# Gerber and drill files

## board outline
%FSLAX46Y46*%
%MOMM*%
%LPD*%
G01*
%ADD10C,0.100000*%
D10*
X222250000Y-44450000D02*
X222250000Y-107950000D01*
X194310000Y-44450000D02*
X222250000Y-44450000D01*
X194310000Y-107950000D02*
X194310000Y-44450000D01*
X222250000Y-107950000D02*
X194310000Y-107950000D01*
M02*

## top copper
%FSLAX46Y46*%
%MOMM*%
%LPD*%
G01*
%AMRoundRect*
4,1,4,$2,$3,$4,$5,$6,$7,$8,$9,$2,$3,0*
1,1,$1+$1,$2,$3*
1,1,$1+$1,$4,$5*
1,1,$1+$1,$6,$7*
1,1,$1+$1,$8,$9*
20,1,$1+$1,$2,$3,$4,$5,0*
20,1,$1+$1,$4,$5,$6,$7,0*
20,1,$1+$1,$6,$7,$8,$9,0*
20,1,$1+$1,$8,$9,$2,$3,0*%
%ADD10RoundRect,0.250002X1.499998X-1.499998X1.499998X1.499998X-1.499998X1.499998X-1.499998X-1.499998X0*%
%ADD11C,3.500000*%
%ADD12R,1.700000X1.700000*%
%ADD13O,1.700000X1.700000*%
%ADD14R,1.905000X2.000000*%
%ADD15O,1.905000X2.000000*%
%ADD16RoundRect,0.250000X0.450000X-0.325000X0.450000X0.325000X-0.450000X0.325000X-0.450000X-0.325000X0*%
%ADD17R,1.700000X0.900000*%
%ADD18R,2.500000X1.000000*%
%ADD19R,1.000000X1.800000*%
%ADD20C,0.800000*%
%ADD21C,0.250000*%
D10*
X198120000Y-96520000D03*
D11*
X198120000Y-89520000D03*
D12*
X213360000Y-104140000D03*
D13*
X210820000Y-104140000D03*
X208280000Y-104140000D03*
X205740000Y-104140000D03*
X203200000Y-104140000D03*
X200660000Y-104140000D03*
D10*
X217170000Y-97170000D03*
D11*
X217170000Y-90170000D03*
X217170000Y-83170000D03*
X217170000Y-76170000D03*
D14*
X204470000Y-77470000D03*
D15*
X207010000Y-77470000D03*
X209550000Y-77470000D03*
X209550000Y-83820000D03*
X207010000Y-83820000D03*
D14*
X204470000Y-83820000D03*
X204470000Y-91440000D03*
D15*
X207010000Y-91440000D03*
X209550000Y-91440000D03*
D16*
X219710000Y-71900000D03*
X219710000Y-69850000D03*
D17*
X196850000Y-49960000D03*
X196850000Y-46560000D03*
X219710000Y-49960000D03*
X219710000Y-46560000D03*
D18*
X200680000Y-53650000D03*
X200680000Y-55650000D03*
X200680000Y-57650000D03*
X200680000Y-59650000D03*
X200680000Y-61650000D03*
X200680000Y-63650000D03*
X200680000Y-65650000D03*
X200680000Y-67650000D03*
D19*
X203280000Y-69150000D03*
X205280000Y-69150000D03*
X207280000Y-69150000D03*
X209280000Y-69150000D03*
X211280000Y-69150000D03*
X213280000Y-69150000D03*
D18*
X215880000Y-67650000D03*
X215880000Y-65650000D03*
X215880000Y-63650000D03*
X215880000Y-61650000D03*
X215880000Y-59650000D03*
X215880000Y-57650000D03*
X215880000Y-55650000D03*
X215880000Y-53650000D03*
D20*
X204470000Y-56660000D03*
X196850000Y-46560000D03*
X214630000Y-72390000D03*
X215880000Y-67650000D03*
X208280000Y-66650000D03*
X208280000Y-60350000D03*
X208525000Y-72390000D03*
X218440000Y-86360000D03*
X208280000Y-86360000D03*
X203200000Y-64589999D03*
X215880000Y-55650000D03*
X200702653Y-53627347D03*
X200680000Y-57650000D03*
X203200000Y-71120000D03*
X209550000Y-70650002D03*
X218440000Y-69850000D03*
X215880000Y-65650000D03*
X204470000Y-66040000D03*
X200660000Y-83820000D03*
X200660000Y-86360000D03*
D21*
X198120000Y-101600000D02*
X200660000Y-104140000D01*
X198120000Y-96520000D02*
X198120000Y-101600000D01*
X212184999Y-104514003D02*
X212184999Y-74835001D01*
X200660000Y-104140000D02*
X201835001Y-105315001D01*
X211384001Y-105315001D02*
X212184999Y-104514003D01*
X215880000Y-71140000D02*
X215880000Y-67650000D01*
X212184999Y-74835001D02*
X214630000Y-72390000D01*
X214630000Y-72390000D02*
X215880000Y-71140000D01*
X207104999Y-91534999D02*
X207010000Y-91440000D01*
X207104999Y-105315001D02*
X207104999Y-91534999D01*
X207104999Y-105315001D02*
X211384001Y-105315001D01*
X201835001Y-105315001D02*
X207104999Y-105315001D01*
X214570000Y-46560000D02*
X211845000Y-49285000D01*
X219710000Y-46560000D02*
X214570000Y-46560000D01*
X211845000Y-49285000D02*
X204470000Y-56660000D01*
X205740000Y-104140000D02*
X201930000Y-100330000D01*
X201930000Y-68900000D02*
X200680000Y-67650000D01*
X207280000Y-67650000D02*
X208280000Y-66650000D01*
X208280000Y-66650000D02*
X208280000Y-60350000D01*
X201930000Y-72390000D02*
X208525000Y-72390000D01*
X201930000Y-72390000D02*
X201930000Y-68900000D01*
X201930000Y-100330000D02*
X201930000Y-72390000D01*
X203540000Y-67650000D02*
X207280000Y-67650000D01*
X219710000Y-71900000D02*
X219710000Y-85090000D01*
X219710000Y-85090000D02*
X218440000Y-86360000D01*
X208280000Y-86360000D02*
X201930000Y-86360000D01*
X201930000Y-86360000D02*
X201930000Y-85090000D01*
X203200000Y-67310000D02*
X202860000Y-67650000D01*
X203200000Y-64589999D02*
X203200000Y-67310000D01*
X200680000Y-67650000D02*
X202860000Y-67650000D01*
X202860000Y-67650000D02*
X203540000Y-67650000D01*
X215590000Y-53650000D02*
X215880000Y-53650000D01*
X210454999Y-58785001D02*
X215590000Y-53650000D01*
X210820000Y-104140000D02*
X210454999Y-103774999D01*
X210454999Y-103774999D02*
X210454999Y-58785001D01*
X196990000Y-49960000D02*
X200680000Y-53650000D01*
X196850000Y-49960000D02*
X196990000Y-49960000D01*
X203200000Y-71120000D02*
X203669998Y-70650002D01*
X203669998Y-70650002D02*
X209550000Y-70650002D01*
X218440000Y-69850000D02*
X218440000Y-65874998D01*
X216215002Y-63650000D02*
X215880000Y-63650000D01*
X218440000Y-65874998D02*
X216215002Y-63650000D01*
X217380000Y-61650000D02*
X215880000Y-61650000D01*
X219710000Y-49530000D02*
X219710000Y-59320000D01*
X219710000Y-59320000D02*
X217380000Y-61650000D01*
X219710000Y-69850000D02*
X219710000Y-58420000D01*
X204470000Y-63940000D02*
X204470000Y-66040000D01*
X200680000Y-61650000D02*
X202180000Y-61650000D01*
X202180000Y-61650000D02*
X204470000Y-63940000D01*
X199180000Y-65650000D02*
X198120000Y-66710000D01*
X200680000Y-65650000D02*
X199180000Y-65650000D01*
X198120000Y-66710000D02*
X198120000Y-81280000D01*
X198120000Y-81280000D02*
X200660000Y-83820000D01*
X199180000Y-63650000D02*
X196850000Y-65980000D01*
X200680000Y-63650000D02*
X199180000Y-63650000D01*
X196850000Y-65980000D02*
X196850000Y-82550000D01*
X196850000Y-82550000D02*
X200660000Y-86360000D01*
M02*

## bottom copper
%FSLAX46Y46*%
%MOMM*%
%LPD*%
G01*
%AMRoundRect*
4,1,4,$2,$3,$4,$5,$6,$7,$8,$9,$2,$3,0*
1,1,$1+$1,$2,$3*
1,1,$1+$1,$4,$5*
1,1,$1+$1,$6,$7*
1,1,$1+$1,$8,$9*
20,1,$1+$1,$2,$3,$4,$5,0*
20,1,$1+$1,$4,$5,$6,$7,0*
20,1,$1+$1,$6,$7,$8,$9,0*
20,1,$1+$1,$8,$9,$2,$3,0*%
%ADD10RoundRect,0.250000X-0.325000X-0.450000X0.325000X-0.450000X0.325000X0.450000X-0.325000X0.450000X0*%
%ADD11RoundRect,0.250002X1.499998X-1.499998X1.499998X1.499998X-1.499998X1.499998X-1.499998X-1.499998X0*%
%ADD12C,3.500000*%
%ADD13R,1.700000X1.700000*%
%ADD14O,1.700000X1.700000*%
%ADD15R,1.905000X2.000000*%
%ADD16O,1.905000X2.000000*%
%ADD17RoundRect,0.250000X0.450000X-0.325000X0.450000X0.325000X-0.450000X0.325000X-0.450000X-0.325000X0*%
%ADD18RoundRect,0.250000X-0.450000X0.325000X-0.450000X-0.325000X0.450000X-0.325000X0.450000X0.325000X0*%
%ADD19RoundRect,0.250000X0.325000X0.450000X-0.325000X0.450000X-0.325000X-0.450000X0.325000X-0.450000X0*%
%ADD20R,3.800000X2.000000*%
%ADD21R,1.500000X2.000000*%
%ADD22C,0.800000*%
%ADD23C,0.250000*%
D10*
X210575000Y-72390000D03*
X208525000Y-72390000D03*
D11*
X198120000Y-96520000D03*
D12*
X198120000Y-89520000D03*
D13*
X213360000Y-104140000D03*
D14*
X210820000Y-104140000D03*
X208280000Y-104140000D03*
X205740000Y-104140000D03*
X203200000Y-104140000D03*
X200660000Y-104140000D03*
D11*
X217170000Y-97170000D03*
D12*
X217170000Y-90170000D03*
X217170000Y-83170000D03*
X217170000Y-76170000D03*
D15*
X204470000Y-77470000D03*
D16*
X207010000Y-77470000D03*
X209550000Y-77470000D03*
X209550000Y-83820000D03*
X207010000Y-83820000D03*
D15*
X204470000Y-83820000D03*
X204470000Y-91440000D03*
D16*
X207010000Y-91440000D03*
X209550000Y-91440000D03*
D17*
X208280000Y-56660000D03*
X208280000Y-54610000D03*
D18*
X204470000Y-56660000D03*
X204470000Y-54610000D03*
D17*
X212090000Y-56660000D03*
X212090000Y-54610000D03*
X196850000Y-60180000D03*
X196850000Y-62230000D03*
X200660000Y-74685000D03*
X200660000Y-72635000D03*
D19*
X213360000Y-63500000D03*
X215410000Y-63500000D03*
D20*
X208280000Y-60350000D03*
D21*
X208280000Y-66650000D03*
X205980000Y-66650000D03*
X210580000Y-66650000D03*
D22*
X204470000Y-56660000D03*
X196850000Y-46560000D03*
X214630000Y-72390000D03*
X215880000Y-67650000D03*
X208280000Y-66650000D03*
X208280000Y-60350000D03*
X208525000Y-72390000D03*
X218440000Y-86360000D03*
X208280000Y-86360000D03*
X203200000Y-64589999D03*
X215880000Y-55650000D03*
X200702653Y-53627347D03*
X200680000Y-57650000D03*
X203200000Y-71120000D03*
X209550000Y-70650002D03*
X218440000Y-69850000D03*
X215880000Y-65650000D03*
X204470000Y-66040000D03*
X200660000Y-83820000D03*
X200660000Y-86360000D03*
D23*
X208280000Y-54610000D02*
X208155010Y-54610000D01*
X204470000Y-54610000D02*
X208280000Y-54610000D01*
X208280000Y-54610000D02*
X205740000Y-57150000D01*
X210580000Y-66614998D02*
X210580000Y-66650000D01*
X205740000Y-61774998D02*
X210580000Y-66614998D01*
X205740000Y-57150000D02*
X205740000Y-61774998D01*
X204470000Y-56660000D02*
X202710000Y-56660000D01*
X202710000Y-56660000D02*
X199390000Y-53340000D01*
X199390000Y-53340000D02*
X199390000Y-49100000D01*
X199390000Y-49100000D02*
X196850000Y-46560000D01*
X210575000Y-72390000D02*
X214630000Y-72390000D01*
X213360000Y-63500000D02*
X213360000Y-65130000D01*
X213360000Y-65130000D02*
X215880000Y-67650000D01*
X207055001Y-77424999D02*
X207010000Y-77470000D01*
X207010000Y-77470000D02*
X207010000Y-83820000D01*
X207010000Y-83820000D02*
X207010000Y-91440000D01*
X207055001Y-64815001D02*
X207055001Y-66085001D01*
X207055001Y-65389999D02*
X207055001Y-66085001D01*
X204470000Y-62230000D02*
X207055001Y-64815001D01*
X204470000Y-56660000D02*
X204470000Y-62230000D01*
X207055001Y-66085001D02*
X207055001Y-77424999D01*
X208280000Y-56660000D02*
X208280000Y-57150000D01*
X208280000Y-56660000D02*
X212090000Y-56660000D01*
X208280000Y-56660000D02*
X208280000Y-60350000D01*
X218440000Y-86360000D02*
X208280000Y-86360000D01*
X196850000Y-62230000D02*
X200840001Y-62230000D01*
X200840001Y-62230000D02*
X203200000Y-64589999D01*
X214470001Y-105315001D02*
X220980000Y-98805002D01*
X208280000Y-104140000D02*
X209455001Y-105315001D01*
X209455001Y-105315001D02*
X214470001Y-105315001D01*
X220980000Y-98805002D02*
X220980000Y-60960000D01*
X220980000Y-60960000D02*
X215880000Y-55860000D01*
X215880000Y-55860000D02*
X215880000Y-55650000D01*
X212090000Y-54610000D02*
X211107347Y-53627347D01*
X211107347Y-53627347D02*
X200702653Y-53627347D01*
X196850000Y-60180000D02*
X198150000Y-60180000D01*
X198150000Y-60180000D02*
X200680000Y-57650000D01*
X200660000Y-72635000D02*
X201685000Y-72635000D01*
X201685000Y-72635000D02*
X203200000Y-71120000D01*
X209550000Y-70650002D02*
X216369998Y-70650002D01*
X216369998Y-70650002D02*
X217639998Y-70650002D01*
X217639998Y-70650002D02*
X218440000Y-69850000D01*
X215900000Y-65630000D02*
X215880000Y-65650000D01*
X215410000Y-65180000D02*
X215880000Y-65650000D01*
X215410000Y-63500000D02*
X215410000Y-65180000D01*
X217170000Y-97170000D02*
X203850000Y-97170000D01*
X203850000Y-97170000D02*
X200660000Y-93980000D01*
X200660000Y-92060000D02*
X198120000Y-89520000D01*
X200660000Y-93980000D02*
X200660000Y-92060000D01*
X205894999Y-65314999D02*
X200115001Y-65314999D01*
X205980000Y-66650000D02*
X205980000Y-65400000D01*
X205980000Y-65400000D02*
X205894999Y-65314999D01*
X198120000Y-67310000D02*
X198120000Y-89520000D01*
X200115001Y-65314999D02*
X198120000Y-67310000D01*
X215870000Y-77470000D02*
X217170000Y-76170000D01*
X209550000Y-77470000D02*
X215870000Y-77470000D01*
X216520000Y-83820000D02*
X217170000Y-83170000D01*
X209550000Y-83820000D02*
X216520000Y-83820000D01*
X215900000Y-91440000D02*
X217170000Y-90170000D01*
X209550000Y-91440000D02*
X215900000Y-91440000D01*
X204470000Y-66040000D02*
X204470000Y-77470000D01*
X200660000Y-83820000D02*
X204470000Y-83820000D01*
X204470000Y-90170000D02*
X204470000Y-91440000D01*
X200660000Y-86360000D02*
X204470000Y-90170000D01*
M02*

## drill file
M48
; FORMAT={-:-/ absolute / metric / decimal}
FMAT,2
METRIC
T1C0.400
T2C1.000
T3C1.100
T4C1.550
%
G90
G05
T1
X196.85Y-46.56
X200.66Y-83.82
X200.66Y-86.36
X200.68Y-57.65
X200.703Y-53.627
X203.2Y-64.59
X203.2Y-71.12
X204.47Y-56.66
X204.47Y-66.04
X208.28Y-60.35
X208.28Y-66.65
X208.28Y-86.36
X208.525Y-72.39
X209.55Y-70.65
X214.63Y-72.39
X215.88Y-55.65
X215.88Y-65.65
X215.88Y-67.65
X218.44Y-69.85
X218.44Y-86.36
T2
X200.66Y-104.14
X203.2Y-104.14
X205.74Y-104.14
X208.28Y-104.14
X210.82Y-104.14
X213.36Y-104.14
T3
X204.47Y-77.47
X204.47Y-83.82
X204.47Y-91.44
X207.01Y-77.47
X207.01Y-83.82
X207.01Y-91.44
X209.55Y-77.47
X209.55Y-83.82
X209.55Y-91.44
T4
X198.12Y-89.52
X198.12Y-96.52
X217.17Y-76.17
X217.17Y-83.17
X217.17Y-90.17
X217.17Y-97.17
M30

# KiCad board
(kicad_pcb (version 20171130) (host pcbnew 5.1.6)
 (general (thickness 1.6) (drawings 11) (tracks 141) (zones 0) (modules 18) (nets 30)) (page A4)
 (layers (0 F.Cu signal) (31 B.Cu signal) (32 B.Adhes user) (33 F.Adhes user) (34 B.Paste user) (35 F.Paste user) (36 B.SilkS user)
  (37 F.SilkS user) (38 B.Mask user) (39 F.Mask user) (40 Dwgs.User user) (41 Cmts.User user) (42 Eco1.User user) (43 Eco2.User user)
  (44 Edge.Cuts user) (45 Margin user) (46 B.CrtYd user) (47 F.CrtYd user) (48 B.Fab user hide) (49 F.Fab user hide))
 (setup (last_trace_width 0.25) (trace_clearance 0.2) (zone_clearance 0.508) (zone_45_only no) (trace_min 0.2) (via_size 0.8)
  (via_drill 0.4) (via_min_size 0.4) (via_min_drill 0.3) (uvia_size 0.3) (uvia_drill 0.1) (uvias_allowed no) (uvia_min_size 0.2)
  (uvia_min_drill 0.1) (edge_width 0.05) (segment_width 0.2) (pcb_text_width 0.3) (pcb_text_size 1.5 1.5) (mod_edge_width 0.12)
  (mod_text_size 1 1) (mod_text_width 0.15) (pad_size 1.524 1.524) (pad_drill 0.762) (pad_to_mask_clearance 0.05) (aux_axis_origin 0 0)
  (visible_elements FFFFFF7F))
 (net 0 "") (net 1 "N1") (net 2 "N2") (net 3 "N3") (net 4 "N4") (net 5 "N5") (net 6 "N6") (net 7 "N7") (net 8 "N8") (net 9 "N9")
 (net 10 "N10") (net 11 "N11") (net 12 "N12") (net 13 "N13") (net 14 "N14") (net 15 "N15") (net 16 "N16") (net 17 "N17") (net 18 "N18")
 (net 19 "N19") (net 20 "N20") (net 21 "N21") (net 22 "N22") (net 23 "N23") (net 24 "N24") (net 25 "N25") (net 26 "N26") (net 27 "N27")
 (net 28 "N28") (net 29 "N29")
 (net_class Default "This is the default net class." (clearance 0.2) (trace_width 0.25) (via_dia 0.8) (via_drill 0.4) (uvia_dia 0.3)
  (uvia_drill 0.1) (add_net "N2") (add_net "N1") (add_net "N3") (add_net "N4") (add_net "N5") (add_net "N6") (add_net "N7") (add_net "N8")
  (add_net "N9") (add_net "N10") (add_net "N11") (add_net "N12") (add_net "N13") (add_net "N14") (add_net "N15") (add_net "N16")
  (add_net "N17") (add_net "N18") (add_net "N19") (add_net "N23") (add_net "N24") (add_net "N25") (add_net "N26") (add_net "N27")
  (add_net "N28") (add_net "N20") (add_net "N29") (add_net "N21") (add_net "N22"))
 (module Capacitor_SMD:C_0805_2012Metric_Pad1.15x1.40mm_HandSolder (layer B.Cu) (at 209.55 72.39)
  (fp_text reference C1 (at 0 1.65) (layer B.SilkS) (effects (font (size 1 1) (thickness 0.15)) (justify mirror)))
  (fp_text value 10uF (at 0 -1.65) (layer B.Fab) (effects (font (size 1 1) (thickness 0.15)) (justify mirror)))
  (pad 2 smd roundrect (at 1.025 0) (size 1.15 1.4) (layers B.Cu B.Paste B.Mask) (roundrect_rratio 0.217391) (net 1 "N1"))
  (pad 1 smd roundrect (at -1.025 0) (size 1.15 1.4) (layers B.Cu B.Paste B.Mask) (roundrect_rratio 0.217391) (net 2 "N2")))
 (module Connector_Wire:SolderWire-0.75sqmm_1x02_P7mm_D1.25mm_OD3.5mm (layer F.Cu) (at 198.12 96.52 90)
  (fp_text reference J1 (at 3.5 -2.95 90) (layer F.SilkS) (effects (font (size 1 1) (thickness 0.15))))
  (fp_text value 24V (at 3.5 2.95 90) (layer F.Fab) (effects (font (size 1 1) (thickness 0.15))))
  (pad 1 thru_hole roundrect (at 0 0 90) (size 3.5 3.5) (drill 1.55) (layers *.Cu *.Mask) (roundrect_rratio 0.07142900000000001)
   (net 1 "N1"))
  (pad 2 thru_hole circle (at 7 0 90) (size 3.5 3.5) (drill 1.55) (layers *.Cu *.Mask) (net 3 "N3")))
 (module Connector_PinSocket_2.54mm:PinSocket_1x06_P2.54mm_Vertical (layer F.Cu) (at 213.36 104.14 270)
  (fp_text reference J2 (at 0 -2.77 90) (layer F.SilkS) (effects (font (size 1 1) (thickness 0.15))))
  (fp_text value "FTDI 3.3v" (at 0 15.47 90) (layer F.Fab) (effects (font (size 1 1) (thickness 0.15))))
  (pad 1 thru_hole rect (at 0 0 270) (size 1.7 1.7) (drill 1) (layers *.Cu *.Mask) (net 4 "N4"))
  (pad 2 thru_hole oval (at 0 2.54 270) (size 1.7 1.7) (drill 1) (layers *.Cu *.Mask) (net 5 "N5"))
  (pad 3 thru_hole oval (at 0 5.08 270) (size 1.7 1.7) (drill 1) (layers *.Cu *.Mask) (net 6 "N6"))
  (pad 4 thru_hole oval (at 0 7.62 270) (size 1.7 1.7) (drill 1) (layers *.Cu *.Mask) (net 2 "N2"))
  (pad 5 thru_hole oval (at 0 10.16 270) (size 1.7 1.7) (drill 1) (layers *.Cu *.Mask) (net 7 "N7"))
  (pad 6 thru_hole oval (at 0 12.7 270) (size 1.7 1.7) (drill 1) (layers *.Cu *.Mask) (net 1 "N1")))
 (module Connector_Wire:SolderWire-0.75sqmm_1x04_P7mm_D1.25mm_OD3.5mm (layer F.Cu) (at 217.17 97.17 90)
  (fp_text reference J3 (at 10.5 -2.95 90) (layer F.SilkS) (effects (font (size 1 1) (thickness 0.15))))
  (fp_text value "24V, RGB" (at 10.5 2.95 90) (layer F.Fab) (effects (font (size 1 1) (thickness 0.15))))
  (pad 1 thru_hole roundrect (at 0 0 90) (size 3.5 3.5) (drill 1.55) (layers *.Cu *.Mask) (roundrect_rratio 0.07142900000000001)
   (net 3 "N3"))
  (pad 2 thru_hole circle (at 7 0 90) (size 3.5 3.5) (drill 1.55) (layers *.Cu *.Mask) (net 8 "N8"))
  (pad 3 thru_hole circle (at 14 0 90) (size 3.5 3.5) (drill 1.55) (layers *.Cu *.Mask) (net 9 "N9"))
  (pad 4 thru_hole circle (at 21 0 90) (size 3.5 3.5) (drill 1.55) (layers *.Cu *.Mask) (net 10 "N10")))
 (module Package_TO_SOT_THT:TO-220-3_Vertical (layer F.Cu) (at 204.47 77.47)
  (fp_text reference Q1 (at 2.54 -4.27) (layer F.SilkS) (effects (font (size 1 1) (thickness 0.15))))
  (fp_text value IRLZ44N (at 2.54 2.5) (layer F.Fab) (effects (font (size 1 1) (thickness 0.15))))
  (pad 1 thru_hole rect (at 0 0) (size 1.905 2) (drill 1.1) (layers *.Cu *.Mask) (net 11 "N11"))
  (pad 2 thru_hole oval (at 2.54 0) (size 1.905 2) (drill 1.1) (layers *.Cu *.Mask) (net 1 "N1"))
  (pad 3 thru_hole oval (at 5.08 0) (size 1.905 2) (drill 1.1) (layers *.Cu *.Mask) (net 10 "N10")))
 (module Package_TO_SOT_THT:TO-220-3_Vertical (layer F.Cu) (at 204.47 83.82)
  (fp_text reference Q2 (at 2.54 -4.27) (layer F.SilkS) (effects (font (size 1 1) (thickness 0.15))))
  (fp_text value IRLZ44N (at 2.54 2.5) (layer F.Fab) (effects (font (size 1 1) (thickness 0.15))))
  (pad 3 thru_hole oval (at 5.08 0) (size 1.905 2) (drill 1.1) (layers *.Cu *.Mask) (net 9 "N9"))
  (pad 2 thru_hole oval (at 2.54 0) (size 1.905 2) (drill 1.1) (layers *.Cu *.Mask) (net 1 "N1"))
  (pad 1 thru_hole rect (at 0 0) (size 1.905 2) (drill 1.1) (layers *.Cu *.Mask) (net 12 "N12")))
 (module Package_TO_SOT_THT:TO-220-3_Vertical (layer F.Cu) (at 204.47 91.44)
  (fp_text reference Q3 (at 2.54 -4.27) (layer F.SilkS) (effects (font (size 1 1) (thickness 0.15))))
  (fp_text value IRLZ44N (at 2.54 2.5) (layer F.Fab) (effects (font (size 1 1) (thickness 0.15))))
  (pad 1 thru_hole rect (at 0 0) (size 1.905 2) (drill 1.1) (layers *.Cu *.Mask) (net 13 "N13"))
  (pad 2 thru_hole oval (at 2.54 0) (size 1.905 2) (drill 1.1) (layers *.Cu *.Mask) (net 1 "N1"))
  (pad 3 thru_hole oval (at 5.08 0) (size 1.905 2) (drill 1.1) (layers *.Cu *.Mask) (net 8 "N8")))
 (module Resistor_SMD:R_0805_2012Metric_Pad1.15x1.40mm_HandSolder (layer B.Cu) (at 208.28 55.635 90)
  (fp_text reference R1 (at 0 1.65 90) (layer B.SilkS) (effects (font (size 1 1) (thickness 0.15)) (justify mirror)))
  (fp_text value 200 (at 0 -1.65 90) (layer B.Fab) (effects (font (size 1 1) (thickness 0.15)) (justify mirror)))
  (pad 1 smd roundrect (at -1.025 0 90) (size 1.15 1.4) (layers B.Cu B.Paste B.Mask) (roundrect_rratio 0.217391) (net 2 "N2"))
  (pad 2 smd roundrect (at 1.025 0 90) (size 1.15 1.4) (layers B.Cu B.Paste B.Mask) (roundrect_rratio 0.217391) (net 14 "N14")))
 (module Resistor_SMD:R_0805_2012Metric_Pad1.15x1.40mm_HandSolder (layer B.Cu) (at 204.47 55.635 270)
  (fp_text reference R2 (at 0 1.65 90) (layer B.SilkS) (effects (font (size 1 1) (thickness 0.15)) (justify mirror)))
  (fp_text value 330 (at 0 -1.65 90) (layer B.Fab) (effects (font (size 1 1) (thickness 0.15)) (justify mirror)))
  (pad 2 smd roundrect (at 1.025 0 270) (size 1.15 1.4) (layers B.Cu B.Paste B.Mask) (roundrect_rratio 0.217391) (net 1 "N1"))
  (pad 1 smd roundrect (at -1.025 0 270) (size 1.15 1.4) (layers B.Cu B.Paste B.Mask) (roundrect_rratio 0.217391) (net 14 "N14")))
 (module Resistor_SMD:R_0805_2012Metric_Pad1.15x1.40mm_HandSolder (layer B.Cu) (at 212.09 55.635 90)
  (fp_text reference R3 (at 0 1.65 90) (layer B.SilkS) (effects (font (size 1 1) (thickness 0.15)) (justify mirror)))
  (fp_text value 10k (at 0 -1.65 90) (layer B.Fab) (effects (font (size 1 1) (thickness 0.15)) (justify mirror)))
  (pad 1 smd roundrect (at -1.025 0 90) (size 1.15 1.4) (layers B.Cu B.Paste B.Mask) (roundrect_rratio 0.217391) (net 2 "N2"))
  (pad 2 smd roundrect (at 1.025 0 90) (size 1.15 1.4) (layers B.Cu B.Paste B.Mask) (roundrect_rratio 0.217391) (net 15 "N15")))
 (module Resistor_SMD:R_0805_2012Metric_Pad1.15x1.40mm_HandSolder (layer B.Cu) (at 196.85 61.205 90)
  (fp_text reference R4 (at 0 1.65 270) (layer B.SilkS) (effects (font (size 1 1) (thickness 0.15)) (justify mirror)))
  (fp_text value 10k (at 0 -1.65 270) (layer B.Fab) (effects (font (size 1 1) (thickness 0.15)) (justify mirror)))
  (pad 2 smd roundrect (at 1.025 0 90) (size 1.15 1.4) (layers B.Cu B.Paste B.Mask) (roundrect_rratio 0.217391) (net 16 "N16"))
  (pad 1 smd roundrect (at -1.025 0 90) (size 1.15 1.4) (layers B.Cu B.Paste B.Mask) (roundrect_rratio 0.217391) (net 2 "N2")))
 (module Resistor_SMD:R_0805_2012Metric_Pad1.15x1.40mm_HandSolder (layer B.Cu) (at 200.66 73.66 90)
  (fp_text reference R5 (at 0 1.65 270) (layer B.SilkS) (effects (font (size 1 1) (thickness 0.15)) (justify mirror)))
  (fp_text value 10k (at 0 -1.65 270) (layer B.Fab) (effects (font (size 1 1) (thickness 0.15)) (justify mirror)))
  (pad 1 smd roundrect (at -1.025 0 90) (size 1.15 1.4) (layers B.Cu B.Paste B.Mask) (roundrect_rratio 0.217391) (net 2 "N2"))
  (pad 2 smd roundrect (at 1.025 0 90) (size 1.15 1.4) (layers B.Cu B.Paste B.Mask) (roundrect_rratio 0.217391) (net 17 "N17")))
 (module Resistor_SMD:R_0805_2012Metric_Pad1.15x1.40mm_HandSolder (layer B.Cu) (at 214.385 63.5 180)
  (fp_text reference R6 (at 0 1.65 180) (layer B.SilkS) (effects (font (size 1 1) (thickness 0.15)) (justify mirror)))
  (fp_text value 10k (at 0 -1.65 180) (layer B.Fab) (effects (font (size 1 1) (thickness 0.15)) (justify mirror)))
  (pad 2 smd roundrect (at 1.025 0 180) (size 1.15 1.4) (layers B.Cu B.Paste B.Mask) (roundrect_rratio 0.217391) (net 1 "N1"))
  (pad 1 smd roundrect (at -1.025 0 180) (size 1.15 1.4) (layers B.Cu B.Paste B.Mask) (roundrect_rratio 0.217391) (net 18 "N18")))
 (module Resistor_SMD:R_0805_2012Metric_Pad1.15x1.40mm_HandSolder (layer F.Cu) (at 219.71 70.875 90)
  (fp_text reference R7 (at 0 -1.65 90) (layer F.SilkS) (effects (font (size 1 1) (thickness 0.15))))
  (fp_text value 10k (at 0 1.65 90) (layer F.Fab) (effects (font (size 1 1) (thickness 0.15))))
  (pad 1 smd roundrect (at -1.025 0 90) (size 1.15 1.4) (layers F.Cu F.Paste F.Mask) (roundrect_rratio 0.217391) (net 2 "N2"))
  (pad 2 smd roundrect (at 1.025 0 90) (size 1.15 1.4) (layers F.Cu F.Paste F.Mask) (roundrect_rratio 0.217391) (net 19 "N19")))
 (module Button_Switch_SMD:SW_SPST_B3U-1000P (layer F.Cu) (at 196.85 48.26 270)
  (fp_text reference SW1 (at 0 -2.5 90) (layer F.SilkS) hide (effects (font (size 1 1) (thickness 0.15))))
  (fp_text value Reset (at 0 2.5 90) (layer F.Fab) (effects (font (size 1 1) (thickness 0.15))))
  (pad 2 smd rect (at 1.7 0 270) (size 0.9 1.7) (layers F.Cu F.Paste F.Mask) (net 15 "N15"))
  (pad 1 smd rect (at -1.7 0 270) (size 0.9 1.7) (layers F.Cu F.Paste F.Mask) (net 1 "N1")))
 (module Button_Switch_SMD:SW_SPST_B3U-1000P (layer F.Cu) (at 219.71 48.26 90)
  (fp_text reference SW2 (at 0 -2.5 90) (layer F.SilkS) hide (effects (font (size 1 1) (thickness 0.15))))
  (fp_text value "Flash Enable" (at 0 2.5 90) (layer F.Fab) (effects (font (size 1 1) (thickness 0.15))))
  (pad 1 smd rect (at -1.7 0 90) (size 0.9 1.7) (layers F.Cu F.Paste F.Mask) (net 19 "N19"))
  (pad 2 smd rect (at 1.7 0 90) (size 0.9 1.7) (layers F.Cu F.Paste F.Mask) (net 1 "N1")))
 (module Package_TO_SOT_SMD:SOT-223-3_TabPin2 (layer B.Cu) (at 208.28 63.5 90)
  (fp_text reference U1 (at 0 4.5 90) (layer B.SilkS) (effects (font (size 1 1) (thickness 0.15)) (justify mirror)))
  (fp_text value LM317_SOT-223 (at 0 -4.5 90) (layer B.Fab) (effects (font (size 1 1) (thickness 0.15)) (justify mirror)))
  (pad 2 smd rect (at 3.15 0 90) (size 2 3.8) (layers B.Cu B.Paste B.Mask) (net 2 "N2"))
  (pad 2 smd rect (at -3.15 0 90) (size 2 1.5) (layers B.Cu B.Paste B.Mask) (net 2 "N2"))
  (pad 3 smd rect (at -3.15 -2.3 90) (size 2 1.5) (layers B.Cu B.Paste B.Mask) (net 3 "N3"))
  (pad 1 smd rect (at -3.15 2.3 90) (size 2 1.5) (layers B.Cu B.Paste B.Mask) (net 14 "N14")))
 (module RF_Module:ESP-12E (layer F.Cu) (at 208.28 57.15)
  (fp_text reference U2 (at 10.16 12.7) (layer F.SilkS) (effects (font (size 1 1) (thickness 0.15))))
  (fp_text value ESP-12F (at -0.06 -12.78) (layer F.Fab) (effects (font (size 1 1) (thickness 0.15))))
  (pad 1 smd rect (at -7.6 -3.5) (size 2.5 1) (layers F.Cu F.Paste F.Mask) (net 15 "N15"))
  (pad 2 smd rect (at -7.6 -1.5) (size 2.5 1) (layers F.Cu F.Paste F.Mask) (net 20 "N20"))
  (pad 3 smd rect (at -7.6 0.5) (size 2.5 1) (layers F.Cu F.Paste F.Mask) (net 16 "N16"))
  (pad 4 smd rect (at -7.6 2.5) (size 2.5 1) (layers F.Cu F.Paste F.Mask) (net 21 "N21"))
  (pad 5 smd rect (at -7.6 4.5) (size 2.5 1) (layers F.Cu F.Paste F.Mask) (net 11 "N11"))
  (pad 6 smd rect (at -7.6 6.5) (size 2.5 1) (layers F.Cu F.Paste F.Mask) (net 13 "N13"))
  (pad 7 smd rect (at -7.6 8.5) (size 2.5 1) (layers F.Cu F.Paste F.Mask) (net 12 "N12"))
  (pad 8 smd rect (at -7.6 10.5) (size 2.5 1) (layers F.Cu F.Paste F.Mask) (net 2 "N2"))
  (pad 9 smd rect (at -5 12) (size 1 1.8) (layers F.Cu F.Paste F.Mask) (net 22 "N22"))
  (pad 10 smd rect (at -3 12) (size 1 1.8) (layers F.Cu F.Paste F.Mask) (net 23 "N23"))
  (pad 11 smd rect (at -1 12) (size 1 1.8) (layers F.Cu F.Paste F.Mask) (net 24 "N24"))
  (pad 12 smd rect (at 1 12) (size 1 1.8) (layers F.Cu F.Paste F.Mask) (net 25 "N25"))
  (pad 13 smd rect (at 3 12) (size 1 1.8) (layers F.Cu F.Paste F.Mask) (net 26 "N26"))
  (pad 14 smd rect (at 5 12) (size 1 1.8) (layers F.Cu F.Paste F.Mask) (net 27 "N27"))
  (pad 15 smd rect (at 7.6 10.5) (size 2.5 1) (layers F.Cu F.Paste F.Mask) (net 1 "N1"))
  (pad 16 smd rect (at 7.6 8.5) (size 2.5 1) (layers F.Cu F.Paste F.Mask) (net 18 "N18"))
  (pad 17 smd rect (at 7.6 6.5) (size 2.5 1) (layers F.Cu F.Paste F.Mask) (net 17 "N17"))
  (pad 18 smd rect (at 7.6 4.5) (size 2.5 1) (layers F.Cu F.Paste F.Mask) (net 19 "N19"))
  (pad 19 smd rect (at 7.6 2.5) (size 2.5 1) (layers F.Cu F.Paste F.Mask) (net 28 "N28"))
  (pad 20 smd rect (at 7.6 0.5) (size 2.5 1) (layers F.Cu F.Paste F.Mask) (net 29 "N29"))
  (pad 21 smd rect (at 7.6 -1.5) (size 2.5 1) (layers F.Cu F.Paste F.Mask) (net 6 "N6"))
  (pad 22 smd rect (at 7.6 -3.5) (size 2.5 1) (layers F.Cu F.Paste F.Mask) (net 5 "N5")))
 (gr_line (start 222.25 44.45) (end 222.25 107.95) (layer Edge.Cuts) (width 0.1))
 (gr_line (start 194.31 44.45) (end 222.25 44.45) (layer Edge.Cuts) (width 0.1))
 (gr_line (start 194.31 107.95) (end 194.31 44.45) (layer Edge.Cuts) (width 0.1))
 (gr_line (start 222.25 107.95) (end 194.31 107.95) (layer Edge.Cuts) (width 0.1))
 (segment (start 208.28 54.61) (end 208.15501 54.61) (width 0.25) (layer B.Cu) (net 14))
 (segment (start 204.47 54.61) (end 208.28 54.61) (width 0.25) (layer B.Cu) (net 14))
 (segment (start 208.28 54.61) (end 205.74 57.15) (width 0.25) (layer B.Cu) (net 14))
 (segment (start 210.58 66.614998) (end 210.58 66.65) (width 0.25) (layer B.Cu) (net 14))
 (segment (start 205.74 61.774998) (end 210.58 66.614998) (width 0.25) (layer B.Cu) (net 14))
 (segment (start 205.74 57.15) (end 205.74 61.774998) (width 0.25) (layer B.Cu) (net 14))
 (segment (start 198.12 101.6) (end 200.66 104.14) (width 0.25) (layer F.Cu) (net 1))
 (segment (start 198.12 96.52) (end 198.12 101.6) (width 0.25) (layer F.Cu) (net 1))
 (via (at 204.47 56.66) (size 0.8) (drill 0.4) (layers F.Cu B.Cu) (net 1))
 (segment (start 212.184999 104.514003) (end 212.184999 74.835001) (width 0.25) (layer F.Cu) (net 1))
 (segment (start 200.66 104.14) (end 201.835001 105.315001) (width 0.25) (layer F.Cu) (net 1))
 (segment (start 211.384001 105.315001) (end 212.184999 104.514003) (width 0.25) (layer F.Cu) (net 1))
 (segment (start 215.88 71.14) (end 215.88 67.65) (width 0.25) (layer F.Cu) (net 1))
 (segment (start 204.47 56.66) (end 202.71 56.66) (width 0.25) (layer B.Cu) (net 1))
 (segment (start 202.71 56.66) (end 199.39 53.34) (width 0.25) (layer B.Cu) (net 1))
 (via (at 196.85 46.56) (size 0.8) (drill 0.4) (layers F.Cu B.Cu) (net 1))
 (segment (start 199.39 53.34) (end 199.39 49.1) (width 0.25) (layer B.Cu) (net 1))
 (segment (start 199.39 49.1) (end 196.85 46.56) (width 0.25) (layer B.Cu) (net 1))
 (via (at 214.63 72.39) (size 0.8) (drill 0.4) (layers F.Cu B.Cu) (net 1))
 (segment (start 210.575 72.39) (end 214.63 72.39) (width 0.25) (layer B.Cu) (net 1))
 (segment (start 212.184999 74.835001) (end 214.63 72.39) (width 0.25) (layer F.Cu) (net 1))
 (segment (start 214.63 72.39) (end 215.88 71.14) (width 0.25) (layer F.Cu) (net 1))
 (via (at 215.88 67.65) (size 0.8) (drill 0.4) (layers F.Cu B.Cu) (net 1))
 (segment (start 213.36 63.5) (end 213.36 65.13) (width 0.25) (layer B.Cu) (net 1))
 (segment (start 213.36 65.13) (end 215.88 67.65) (width 0.25) (layer B.Cu) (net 1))
 (segment (start 207.055001 77.424999) (end 207.01 77.47) (width 0.25) (layer B.Cu) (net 1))
 (segment (start 207.01 77.47) (end 207.01 83.82) (width 0.25) (layer B.Cu) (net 1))
 (segment (start 207.01 83.82) (end 207.01 91.44) (width 0.25) (layer B.Cu) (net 1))
 (segment (start 207.055001 64.815001) (end 207.055001 66.085001) (width 0.25) (layer B.Cu) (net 1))
 (segment (start 207.055001 65.389999) (end 207.055001 66.085001) (width 0.25) (layer B.Cu) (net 1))
 (segment (start 204.47 62.23) (end 207.055001 64.815001) (width 0.25) (layer B.Cu) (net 1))
 (segment (start 204.47 56.66) (end 204.47 62.23) (width 0.25) (layer B.Cu) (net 1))
 (segment (start 207.055001 66.085001) (end 207.055001 77.424999) (width 0.25) (layer B.Cu) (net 1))
 (segment (start 207.104999 91.534999) (end 207.01 91.44) (width 0.25) (layer F.Cu) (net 1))
 (segment (start 207.104999 105.315001) (end 207.104999 91.534999) (width 0.25) (layer F.Cu) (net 1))
 (segment (start 207.104999 105.315001) (end 211.384001 105.315001) (width 0.25) (layer F.Cu) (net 1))
 (segment (start 201.835001 105.315001) (end 207.104999 105.315001) (width 0.25) (layer F.Cu) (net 1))
 (segment (start 214.57 46.56) (end 211.845 49.285) (width 0.25) (layer F.Cu) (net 1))
 (segment (start 219.71 46.56) (end 214.57 46.56) (width 0.25) (layer F.Cu) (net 1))
 (segment (start 211.845 49.285) (end 204.47 56.66) (width 0.25) (layer F.Cu) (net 1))
 (segment (start 208.28 56.66) (end 208.28 57.15) (width 0.25) (layer B.Cu) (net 2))
 (segment (start 208.28 56.66) (end 212.09 56.66) (width 0.25) (layer B.Cu) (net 2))
 (segment (start 208.28 56.66) (end 208.28 60.35) (width 0.25) (layer B.Cu) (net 2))
 (segment (start 205.74 104.14) (end 201.93 100.33) (width 0.25) (layer F.Cu) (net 2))
 (segment (start 201.93 68.9) (end 200.68 67.65) (width 0.25) (layer F.Cu) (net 2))
 (via (at 208.28 66.65) (size 0.8) (drill 0.4) (layers F.Cu B.Cu) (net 2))
 (segment (start 207.28 67.65) (end 208.28 66.65) (width 0.25) (layer F.Cu) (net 2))
 (via (at 208.28 60.35) (size 0.8) (drill 0.4) (layers F.Cu B.Cu) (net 2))
 (segment (start 208.28 66.65) (end 208.28 60.35) (width 0.25) (layer F.Cu) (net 2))
 (via (at 208.525 72.39) (size 0.8) (drill 0.4) (layers F.Cu B.Cu) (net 2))
 (segment (start 201.93 72.39) (end 208.525 72.39) (width 0.25) (layer F.Cu) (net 2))
 (segment (start 201.93 72.39) (end 201.93 68.9) (width 0.25) (layer F.Cu) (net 2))
 (segment (start 201.93 100.33) (end 201.93 72.39) (width 0.25) (layer F.Cu) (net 2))
 (segment (start 203.54 67.65) (end 207.28 67.65) (width 0.25) (layer F.Cu) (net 2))
 (via (at 218.44 86.36) (size 0.8) (drill 0.4) (layers F.Cu B.Cu) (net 2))
 (segment (start 219.71 71.9) (end 219.71 85.09) (width 0.25) (layer F.Cu) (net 2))
 (segment (start 219.71 85.09) (end 218.44 86.36) (width 0.25) (layer F.Cu) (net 2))
 (via (at 208.28 86.36) (size 0.8) (drill 0.4) (layers F.Cu B.Cu) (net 2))
 (segment (start 218.44 86.36) (end 208.28 86.36) (width 0.25) (layer B.Cu) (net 2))
 (segment (start 208.28 86.36) (end 201.93 86.36) (width 0.25) (layer F.Cu) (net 2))
 (segment (start 201.93 86.36) (end 201.93 85.09) (width 0.25) (layer F.Cu) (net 2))
 (via (at 203.2 64.589999) (size 0.8) (drill 0.4) (layers F.Cu B.Cu) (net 2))
 (segment (start 196.85 62.23) (end 200.840001 62.23) (width 0.25) (layer B.Cu) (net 2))
 (segment (start 200.840001 62.23) (end 203.2 64.589999) (width 0.25) (layer B.Cu) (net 2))
 (segment (start 203.2 67.31) (end 202.86 67.65) (width 0.25) (layer F.Cu) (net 2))
 (segment (start 203.2 64.589999) (end 203.2 67.31) (width 0.25) (layer F.Cu) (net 2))
 (segment (start 200.68 67.65) (end 202.86 67.65) (width 0.25) (layer F.Cu) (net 2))
 (segment (start 202.86 67.65) (end 203.54 67.65) (width 0.25) (layer F.Cu) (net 2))
 (segment (start 214.470001 105.315001) (end 220.98 98.805002) (width 0.25) (layer B.Cu) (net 6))
 (segment (start 208.28 104.14) (end 209.455001 105.315001) (width 0.25) (layer B.Cu) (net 6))
 (segment (start 209.455001 105.315001) (end 214.470001 105.315001) (width 0.25) (layer B.Cu) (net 6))
 (segment (start 220.98 98.805002) (end 220.98 60.96) (width 0.25) (layer B.Cu) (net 6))
 (via (at 215.88 55.65) (size 0.8) (drill 0.4) (layers F.Cu B.Cu) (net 6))
 (segment (start 220.98 60.96) (end 215.88 55.86) (width 0.25) (layer B.Cu) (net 6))
 (segment (start 215.88 55.86) (end 215.88 55.65) (width 0.25) (layer B.Cu) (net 6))
 (segment (start 215.59 53.65) (end 215.88 53.65) (width 0.25) (layer F.Cu) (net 5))
 (segment (start 210.454999 58.785001) (end 215.59 53.65) (width 0.25) (layer F.Cu) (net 5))
 (segment (start 210.82 104.14) (end 210.454999 103.774999) (width 0.25) (layer F.Cu) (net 5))
 (segment (start 210.454999 103.774999) (end 210.454999 58.785001) (width 0.25) (layer F.Cu) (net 5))
 (segment (start 196.99 49.96) (end 200.68 53.65) (width 0.25) (layer F.Cu) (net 15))
 (segment (start 196.85 49.96) (end 196.99 49.96) (width 0.25) (layer F.Cu) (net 15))
 (segment (start 212.09 54.61) (end 211.107347 53.627347) (width 0.25) (layer B.Cu) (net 15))
 (via (at 200.702653 53.627347) (size 0.8) (drill 0.4) (layers F.Cu B.Cu) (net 15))
 (segment (start 211.107347 53.627347) (end 200.702653 53.627347) (width 0.25) (layer B.Cu) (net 15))
 (via (at 200.68 57.65) (size 0.8) (drill 0.4) (layers F.Cu B.Cu) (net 16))
 (segment (start 196.85 60.18) (end 198.15 60.18) (width 0.25) (layer B.Cu) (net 16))
 (segment (start 198.15 60.18) (end 200.68 57.65) (width 0.25) (layer B.Cu) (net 16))
 (via (at 203.2 71.12) (size 0.8) (drill 0.4) (layers F.Cu B.Cu) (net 17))
 (segment (start 200.66 72.635) (end 201.685 72.635) (width 0.25) (layer B.Cu) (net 17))
 (segment (start 201.685 72.635) (end 203.2 71.12) (width 0.25) (layer B.Cu) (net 17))
 (via (at 209.55 70.650002) (size 0.8) (drill 0.4) (layers F.Cu B.Cu) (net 17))
 (segment (start 203.2 71.12) (end 203.669998 70.650002) (width 0.25) (layer F.Cu) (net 17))
 (segment (start 203.669998 70.650002) (end 209.55 70.650002) (width 0.25) (layer F.Cu) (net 17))
 (segment (start 209.55 70.650002) (end 216.369998 70.650002) (width 0.25) (layer B.Cu) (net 17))
 (via (at 218.44 69.85) (size 0.8) (drill 0.4) (layers F.Cu B.Cu) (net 17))
 (segment (start 216.369998 70.650002) (end 217.639998 70.650002) (width 0.25) (layer B.Cu) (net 17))
 (segment (start 217.639998 70.650002) (end 218.44 69.85) (width 0.25) (layer B.Cu) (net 17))
 (segment (start 218.44 69.85) (end 218.44 65.874998) (width 0.25) (layer F.Cu) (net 17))
 (segment (start 216.215002 63.65) (end 215.88 63.65) (width 0.25) (layer F.Cu) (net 17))
 (segment (start 218.44 65.874998) (end 216.215002 63.65) (width 0.25) (layer F.Cu) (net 17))
 (via (at 215.88 65.65) (size 0.8) (drill 0.4) (layers F.Cu B.Cu) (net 18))
 (segment (start 215.9 65.63) (end 215.88 65.65) (width 0.25) (layer B.Cu) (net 18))
 (segment (start 215.41 65.18) (end 215.88 65.65) (width 0.25) (layer B.Cu) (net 18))
 (segment (start 215.41 63.5) (end 215.41 65.18) (width 0.25) (layer B.Cu) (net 18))
 (segment (start 217.38 61.65) (end 215.88 61.65) (width 0.25) (layer F.Cu) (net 19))
 (segment (start 219.71 49.53) (end 219.71 59.32) (width 0.25) (layer F.Cu) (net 19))
 (segment (start 219.71 59.32) (end 217.38 61.65) (width 0.25) (layer F.Cu) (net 19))
 (segment (start 219.71 69.85) (end 219.71 58.42) (width 0.25) (layer F.Cu) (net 19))
 (segment (start 217.17 97.17) (end 203.85 97.17) (width 0.25) (layer B.Cu) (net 3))
 (segment (start 203.85 97.17) (end 200.66 93.98) (width 0.25) (layer B.Cu) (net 3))
 (segment (start 200.66 92.06) (end 198.12 89.52) (width 0.25) (layer B.Cu) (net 3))
 (segment (start 200.66 93.98) (end 200.66 92.06) (width 0.25) (layer B.Cu) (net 3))
 (segment (start 205.894999 65.314999) (end 200.115001 65.314999) (width 0.25) (layer B.Cu) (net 3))
 (segment (start 205.98 66.65) (end 205.98 65.4) (width 0.25) (layer B.Cu) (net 3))
 (segment (start 205.98 65.4) (end 205.894999 65.314999) (width 0.25) (layer B.Cu) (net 3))
 (segment (start 198.12 67.31) (end 198.12 89.52) (width 0.25) (layer B.Cu) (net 3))
 (segment (start 200.115001 65.314999) (end 198.12 67.31) (width 0.25) (layer B.Cu) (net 3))
 (segment (start 215.87 77.47) (end 217.17 76.17) (width 0.25) (layer B.Cu) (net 10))
 (segment (start 209.55 77.47) (end 215.87 77.47) (width 0.25) (layer B.Cu) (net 10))
 (segment (start 216.52 83.82) (end 217.17 83.17) (width 0.25) (layer B.Cu) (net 9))
 (segment (start 209.55 83.82) (end 216.52 83.82) (width 0.25) (layer B.Cu) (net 9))
 (segment (start 215.9 91.44) (end 217.17 90.17) (width 0.25) (layer B.Cu) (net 8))
 (segment (start 209.55 91.44) (end 215.9 91.44) (width 0.25) (layer B.Cu) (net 8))
 (via (at 204.47 66.04) (size 0.8) (drill 0.4) (layers F.Cu B.Cu) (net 11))
 (segment (start 204.47 63.94) (end 204.47 66.04) (width 0.25) (layer F.Cu) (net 11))
 (segment (start 200.68 61.65) (end 202.18 61.65) (width 0.25) (layer F.Cu) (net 11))
 (segment (start 202.18 61.65) (end 204.47 63.94) (width 0.25) (layer F.Cu) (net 11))
 (segment (start 204.47 66.04) (end 204.47 77.47) (width 0.25) (layer B.Cu) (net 11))
 (segment (start 199.18 65.65) (end 198.12 66.71) (width 0.25) (layer F.Cu) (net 12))
 (segment (start 200.68 65.65) (end 199.18 65.65) (width 0.25) (layer F.Cu) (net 12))
 (segment (start 198.12 66.71) (end 198.12 81.28) (width 0.25) (layer F.Cu) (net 12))
 (via (at 200.66 83.82) (size 0.8) (drill 0.4) (layers F.Cu B.Cu) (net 12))
 (segment (start 198.12 81.28) (end 200.66 83.82) (width 0.25) (layer F.Cu) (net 12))
 (segment (start 200.66 83.82) (end 204.47 83.82) (width 0.25) (layer B.Cu) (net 12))
 (segment (start 199.18 63.65) (end 196.85 65.98) (width 0.25) (layer F.Cu) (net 13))
 (segment (start 200.68 63.65) (end 199.18 63.65) (width 0.25) (layer F.Cu) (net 13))
 (via (at 200.66 86.36) (size 0.8) (drill 0.4) (layers F.Cu B.Cu) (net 13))
 (segment (start 196.85 65.98) (end 196.85 82.55) (width 0.25) (layer F.Cu) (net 13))
 (segment (start 196.85 82.55) (end 200.66 86.36) (width 0.25) (layer F.Cu) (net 13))
 (segment (start 204.47 90.17) (end 204.47 91.44) (width 0.25) (layer B.Cu) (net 13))
 (segment (start 200.66 86.36) (end 204.47 90.17) (width 0.25) (layer B.Cu) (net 13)))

